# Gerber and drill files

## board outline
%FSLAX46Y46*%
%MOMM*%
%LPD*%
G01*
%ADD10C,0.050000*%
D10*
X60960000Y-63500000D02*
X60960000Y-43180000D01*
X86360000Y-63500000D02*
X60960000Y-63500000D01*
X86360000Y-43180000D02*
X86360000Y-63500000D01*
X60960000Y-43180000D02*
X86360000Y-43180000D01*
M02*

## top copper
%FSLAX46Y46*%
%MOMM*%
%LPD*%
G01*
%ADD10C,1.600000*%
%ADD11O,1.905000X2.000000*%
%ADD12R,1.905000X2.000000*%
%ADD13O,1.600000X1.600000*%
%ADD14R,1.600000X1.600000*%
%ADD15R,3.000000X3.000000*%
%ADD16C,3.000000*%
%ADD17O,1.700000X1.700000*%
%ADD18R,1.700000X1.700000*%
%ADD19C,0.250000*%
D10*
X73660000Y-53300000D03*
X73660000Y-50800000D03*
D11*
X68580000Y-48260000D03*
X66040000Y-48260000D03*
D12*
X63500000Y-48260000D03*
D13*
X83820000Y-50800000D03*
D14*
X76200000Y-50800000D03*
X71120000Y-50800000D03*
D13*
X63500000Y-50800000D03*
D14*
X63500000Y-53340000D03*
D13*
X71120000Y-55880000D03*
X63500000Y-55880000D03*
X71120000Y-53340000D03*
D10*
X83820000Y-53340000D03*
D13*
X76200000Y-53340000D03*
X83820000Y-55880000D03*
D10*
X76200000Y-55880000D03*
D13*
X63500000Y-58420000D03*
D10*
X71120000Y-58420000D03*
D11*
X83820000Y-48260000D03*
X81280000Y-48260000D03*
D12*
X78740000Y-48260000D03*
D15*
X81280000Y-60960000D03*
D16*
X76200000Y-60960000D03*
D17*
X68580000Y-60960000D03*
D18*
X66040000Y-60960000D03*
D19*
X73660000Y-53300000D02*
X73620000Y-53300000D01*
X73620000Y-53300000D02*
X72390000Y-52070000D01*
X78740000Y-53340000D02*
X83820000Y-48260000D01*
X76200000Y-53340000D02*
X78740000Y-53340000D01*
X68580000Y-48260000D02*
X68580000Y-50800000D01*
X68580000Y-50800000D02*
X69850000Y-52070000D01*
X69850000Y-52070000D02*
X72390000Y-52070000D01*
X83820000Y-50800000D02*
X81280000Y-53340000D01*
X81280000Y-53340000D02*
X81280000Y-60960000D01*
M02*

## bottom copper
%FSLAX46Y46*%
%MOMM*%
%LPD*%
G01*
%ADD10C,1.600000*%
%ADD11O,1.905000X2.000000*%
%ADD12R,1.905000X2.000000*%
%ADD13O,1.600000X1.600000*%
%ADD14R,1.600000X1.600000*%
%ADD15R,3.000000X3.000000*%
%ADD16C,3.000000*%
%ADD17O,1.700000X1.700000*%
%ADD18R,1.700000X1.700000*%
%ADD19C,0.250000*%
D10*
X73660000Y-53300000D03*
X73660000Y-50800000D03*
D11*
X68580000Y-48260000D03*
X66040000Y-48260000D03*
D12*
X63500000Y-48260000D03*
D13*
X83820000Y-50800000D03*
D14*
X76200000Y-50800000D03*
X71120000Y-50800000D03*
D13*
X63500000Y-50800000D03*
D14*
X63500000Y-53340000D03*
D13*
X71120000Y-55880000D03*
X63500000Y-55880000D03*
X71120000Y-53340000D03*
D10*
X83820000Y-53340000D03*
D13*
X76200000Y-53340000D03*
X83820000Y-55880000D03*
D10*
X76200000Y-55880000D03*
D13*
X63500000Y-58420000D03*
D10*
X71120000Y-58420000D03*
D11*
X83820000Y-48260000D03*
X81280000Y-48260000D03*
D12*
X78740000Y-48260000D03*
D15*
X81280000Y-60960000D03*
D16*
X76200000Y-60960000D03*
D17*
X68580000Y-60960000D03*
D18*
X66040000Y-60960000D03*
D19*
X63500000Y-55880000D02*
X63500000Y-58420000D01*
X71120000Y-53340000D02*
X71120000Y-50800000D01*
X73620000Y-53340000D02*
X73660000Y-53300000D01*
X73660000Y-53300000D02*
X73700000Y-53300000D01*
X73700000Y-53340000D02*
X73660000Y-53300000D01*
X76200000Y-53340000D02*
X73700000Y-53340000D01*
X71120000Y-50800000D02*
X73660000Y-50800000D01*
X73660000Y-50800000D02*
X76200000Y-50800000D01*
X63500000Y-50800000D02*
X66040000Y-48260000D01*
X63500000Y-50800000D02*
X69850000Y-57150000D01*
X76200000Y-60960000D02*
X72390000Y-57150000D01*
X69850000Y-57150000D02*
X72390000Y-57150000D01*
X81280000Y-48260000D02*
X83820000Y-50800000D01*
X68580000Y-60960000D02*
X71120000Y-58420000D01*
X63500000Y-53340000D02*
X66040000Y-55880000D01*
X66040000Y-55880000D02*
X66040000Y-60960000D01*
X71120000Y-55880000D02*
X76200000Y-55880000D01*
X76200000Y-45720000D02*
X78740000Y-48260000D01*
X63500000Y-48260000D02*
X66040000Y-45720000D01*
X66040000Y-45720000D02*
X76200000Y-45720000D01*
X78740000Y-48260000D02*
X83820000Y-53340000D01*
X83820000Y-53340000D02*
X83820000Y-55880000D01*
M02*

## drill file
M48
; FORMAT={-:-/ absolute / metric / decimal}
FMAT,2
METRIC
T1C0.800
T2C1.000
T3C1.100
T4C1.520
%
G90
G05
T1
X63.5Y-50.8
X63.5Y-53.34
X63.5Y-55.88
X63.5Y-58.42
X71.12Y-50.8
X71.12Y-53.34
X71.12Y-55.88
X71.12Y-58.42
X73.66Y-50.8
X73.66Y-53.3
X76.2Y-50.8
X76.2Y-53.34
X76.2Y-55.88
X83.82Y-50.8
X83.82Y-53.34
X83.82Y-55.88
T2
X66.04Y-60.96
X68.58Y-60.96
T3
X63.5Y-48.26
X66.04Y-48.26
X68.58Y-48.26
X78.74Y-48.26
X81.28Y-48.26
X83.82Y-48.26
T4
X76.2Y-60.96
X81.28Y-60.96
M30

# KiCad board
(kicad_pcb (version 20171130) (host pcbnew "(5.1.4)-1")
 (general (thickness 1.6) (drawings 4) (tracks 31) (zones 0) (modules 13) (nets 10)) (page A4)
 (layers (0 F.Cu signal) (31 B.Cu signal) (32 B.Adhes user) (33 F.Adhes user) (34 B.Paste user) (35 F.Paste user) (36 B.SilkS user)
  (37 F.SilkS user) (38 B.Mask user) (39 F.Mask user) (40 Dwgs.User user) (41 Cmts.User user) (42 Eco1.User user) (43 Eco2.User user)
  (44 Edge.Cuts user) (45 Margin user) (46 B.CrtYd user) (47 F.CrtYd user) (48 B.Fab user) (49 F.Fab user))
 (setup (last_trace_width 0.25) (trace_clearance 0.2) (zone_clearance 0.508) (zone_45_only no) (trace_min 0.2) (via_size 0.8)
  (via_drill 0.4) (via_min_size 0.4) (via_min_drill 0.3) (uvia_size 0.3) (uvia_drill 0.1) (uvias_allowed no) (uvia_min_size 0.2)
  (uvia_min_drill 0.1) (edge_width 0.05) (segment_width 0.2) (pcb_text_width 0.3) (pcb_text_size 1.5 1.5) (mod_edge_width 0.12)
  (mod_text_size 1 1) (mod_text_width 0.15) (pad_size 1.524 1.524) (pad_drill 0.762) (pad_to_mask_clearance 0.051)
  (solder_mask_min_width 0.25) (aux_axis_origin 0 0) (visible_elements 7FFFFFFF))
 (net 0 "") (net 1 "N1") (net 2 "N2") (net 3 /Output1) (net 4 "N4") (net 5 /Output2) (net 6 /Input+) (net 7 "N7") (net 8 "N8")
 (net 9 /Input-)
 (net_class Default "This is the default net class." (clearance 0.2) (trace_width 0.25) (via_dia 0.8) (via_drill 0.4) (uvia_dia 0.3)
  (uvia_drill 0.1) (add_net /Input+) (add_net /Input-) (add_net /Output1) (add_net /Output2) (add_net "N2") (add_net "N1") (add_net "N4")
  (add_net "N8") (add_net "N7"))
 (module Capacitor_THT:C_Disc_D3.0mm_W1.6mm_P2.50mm (layer F.Cu) (at 73.66 50.8 270)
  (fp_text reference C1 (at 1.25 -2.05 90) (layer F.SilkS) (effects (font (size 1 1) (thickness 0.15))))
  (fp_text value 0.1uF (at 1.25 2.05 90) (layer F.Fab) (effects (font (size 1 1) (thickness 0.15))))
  (pad 2 thru_hole circle (at 2.5 0 270) (size 1.6 1.6) (drill 0.8) (layers *.Cu *.Mask) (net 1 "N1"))
  (pad 1 thru_hole circle (at 0 0 270) (size 1.6 1.6) (drill 0.8) (layers *.Cu *.Mask) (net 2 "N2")))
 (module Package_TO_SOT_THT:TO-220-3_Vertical (layer F.Cu) (at 63.5 48.26)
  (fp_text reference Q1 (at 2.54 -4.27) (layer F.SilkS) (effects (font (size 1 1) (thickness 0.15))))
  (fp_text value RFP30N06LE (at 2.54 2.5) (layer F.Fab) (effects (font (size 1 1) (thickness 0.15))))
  (pad 3 thru_hole oval (at 5.08 0) (size 1.905 2) (drill 1.1) (layers *.Cu *.Mask) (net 1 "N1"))
  (pad 2 thru_hole oval (at 2.54 0) (size 1.905 2) (drill 1.1) (layers *.Cu *.Mask) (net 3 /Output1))
  (pad 1 thru_hole rect (at 0 0) (size 1.905 2) (drill 1.1) (layers *.Cu *.Mask) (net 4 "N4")))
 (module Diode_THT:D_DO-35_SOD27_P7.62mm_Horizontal (layer F.Cu) (at 76.2 50.8)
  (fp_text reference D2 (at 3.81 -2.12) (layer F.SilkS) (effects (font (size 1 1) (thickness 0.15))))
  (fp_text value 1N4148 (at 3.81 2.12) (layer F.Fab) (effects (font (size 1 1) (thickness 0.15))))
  (pad 2 thru_hole oval (at 7.62 0) (size 1.6 1.6) (drill 0.8) (layers *.Cu *.Mask) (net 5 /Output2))
  (pad 1 thru_hole rect (at 0 0) (size 1.6 1.6) (drill 0.8) (layers *.Cu *.Mask) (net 2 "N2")))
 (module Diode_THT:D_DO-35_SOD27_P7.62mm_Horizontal (layer F.Cu) (at 71.12 50.8 180)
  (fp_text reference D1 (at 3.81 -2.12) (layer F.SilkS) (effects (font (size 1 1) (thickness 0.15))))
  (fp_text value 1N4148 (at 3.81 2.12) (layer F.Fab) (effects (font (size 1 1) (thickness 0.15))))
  (pad 1 thru_hole rect (at 0 0 180) (size 1.6 1.6) (drill 0.8) (layers *.Cu *.Mask) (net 2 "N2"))
  (pad 2 thru_hole oval (at 7.62 0 180) (size 1.6 1.6) (drill 0.8) (layers *.Cu *.Mask) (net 3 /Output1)))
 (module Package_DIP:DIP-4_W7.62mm (layer F.Cu) (at 63.5 53.34)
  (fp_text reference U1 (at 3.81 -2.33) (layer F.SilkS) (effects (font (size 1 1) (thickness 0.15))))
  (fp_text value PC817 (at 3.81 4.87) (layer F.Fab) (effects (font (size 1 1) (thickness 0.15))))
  (pad 1 thru_hole rect (at 0 0) (size 1.6 1.6) (drill 0.8) (layers *.Cu *.Mask) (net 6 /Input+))
  (pad 3 thru_hole oval (at 7.62 2.54) (size 1.6 1.6) (drill 0.8) (layers *.Cu *.Mask) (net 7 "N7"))
  (pad 2 thru_hole oval (at 0 2.54) (size 1.6 1.6) (drill 0.8) (layers *.Cu *.Mask) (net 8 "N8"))
  (pad 4 thru_hole oval (at 7.62 0) (size 1.6 1.6) (drill 0.8) (layers *.Cu *.Mask) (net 2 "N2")))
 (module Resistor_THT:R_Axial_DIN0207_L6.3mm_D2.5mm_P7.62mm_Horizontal (layer F.Cu) (at 83.82 53.34 180)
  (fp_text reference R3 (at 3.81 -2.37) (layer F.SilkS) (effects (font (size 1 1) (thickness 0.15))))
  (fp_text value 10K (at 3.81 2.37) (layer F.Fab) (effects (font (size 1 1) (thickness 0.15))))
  (pad 1 thru_hole circle (at 0 0 180) (size 1.6 1.6) (drill 0.8) (layers *.Cu *.Mask) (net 4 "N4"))
  (pad 2 thru_hole oval (at 7.62 0 180) (size 1.6 1.6) (drill 0.8) (layers *.Cu *.Mask) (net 1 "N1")))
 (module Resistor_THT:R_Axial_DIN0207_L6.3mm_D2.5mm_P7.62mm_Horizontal (layer F.Cu) (at 76.2 55.88)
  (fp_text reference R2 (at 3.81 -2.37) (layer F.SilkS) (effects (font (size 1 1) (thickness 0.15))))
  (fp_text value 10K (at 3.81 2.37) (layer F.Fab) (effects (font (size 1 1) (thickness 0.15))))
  (pad 2 thru_hole oval (at 7.62 0) (size 1.6 1.6) (drill 0.8) (layers *.Cu *.Mask) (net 4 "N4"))
  (pad 1 thru_hole circle (at 0 0) (size 1.6 1.6) (drill 0.8) (layers *.Cu *.Mask) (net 7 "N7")))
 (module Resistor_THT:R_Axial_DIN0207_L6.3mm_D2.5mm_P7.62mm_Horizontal (layer F.Cu) (at 71.12 58.42 180)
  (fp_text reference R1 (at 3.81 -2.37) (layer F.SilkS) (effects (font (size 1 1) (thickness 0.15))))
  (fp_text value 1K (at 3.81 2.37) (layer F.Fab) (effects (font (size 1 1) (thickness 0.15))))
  (pad 2 thru_hole oval (at 7.62 0 180) (size 1.6 1.6) (drill 0.8) (layers *.Cu *.Mask) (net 8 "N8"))
  (pad 1 thru_hole circle (at 0 0 180) (size 1.6 1.6) (drill 0.8) (layers *.Cu *.Mask) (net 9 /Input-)))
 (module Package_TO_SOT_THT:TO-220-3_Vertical (layer F.Cu) (at 78.74 48.26)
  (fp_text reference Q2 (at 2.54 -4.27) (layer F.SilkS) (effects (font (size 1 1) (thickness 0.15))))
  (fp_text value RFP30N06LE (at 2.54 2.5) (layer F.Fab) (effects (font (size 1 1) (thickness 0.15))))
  (pad 3 thru_hole oval (at 5.08 0) (size 1.905 2) (drill 1.1) (layers *.Cu *.Mask) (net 1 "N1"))
  (pad 2 thru_hole oval (at 2.54 0) (size 1.905 2) (drill 1.1) (layers *.Cu *.Mask) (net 5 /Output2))
  (pad 1 thru_hole rect (at 0 0) (size 1.905 2) (drill 1.1) (layers *.Cu *.Mask) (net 4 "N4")))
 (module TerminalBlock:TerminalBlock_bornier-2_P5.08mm (layer F.Cu) (at 81.28 60.96 180)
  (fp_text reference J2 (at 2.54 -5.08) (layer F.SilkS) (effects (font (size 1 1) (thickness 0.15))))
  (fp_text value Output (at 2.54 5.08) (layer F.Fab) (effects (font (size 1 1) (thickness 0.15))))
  (pad 1 thru_hole rect (at 0 0 180) (size 3 3) (drill 1.52) (layers *.Cu *.Mask) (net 5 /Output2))
  (pad 2 thru_hole circle (at 5.08 0 180) (size 3 3) (drill 1.52) (layers *.Cu *.Mask) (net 3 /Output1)))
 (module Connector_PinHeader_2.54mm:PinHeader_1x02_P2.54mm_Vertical (layer F.Cu) (at 66.04 60.96 90)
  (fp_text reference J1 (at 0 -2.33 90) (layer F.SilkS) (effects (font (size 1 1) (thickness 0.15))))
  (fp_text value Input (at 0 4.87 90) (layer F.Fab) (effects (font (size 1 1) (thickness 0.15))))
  (pad 2 thru_hole oval (at 0 2.54 90) (size 1.7 1.7) (drill 1) (layers *.Cu *.Mask) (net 9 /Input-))
  (pad 1 thru_hole rect (at 0 0 90) (size 1.7 1.7) (drill 1) (layers *.Cu *.Mask) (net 6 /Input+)))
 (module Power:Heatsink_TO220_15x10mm (layer F.Cu) (at 81.28 44.45)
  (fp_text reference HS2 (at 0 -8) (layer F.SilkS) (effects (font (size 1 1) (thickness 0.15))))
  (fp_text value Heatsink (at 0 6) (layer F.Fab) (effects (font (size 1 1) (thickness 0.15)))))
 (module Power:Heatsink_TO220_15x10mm (layer F.Cu) (at 66.04 44.45)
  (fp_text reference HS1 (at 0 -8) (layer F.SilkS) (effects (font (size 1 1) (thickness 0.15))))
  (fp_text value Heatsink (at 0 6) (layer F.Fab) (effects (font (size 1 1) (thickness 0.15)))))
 (gr_line (start 60.96 63.5) (end 60.96 43.18) (layer Edge.Cuts) (width 0.05))
 (gr_line (start 86.36 63.5) (end 60.96 63.5) (layer Edge.Cuts) (width 0.05))
 (gr_line (start 86.36 43.18) (end 86.36 63.5) (layer Edge.Cuts) (width 0.05))
 (gr_line (start 60.96 43.18) (end 86.36 43.18) (layer Edge.Cuts) (width 0.05))
 (segment (start 63.5 55.88) (end 63.5 58.42) (width 0.25) (layer B.Cu) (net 8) (status 30))
 (segment (start 71.12 53.34) (end 71.12 50.8) (width 0.25) (layer B.Cu) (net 2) (status 30))
 (segment (start 73.62 53.34) (end 73.66 53.3) (width 0.25) (layer B.Cu) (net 1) (status 30))
 (segment (start 73.66 53.3) (end 73.7 53.3) (width 0.25) (layer B.Cu) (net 1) (status 30))
 (segment (start 73.7 53.34) (end 73.66 53.3) (width 0.25) (layer B.Cu) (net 1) (status 30))
 (segment (start 76.2 53.34) (end 73.7 53.34) (width 0.25) (layer B.Cu) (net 1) (status 30))
 (segment (start 73.66 53.3) (end 73.62 53.3) (width 0.25) (layer F.Cu) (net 1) (status 30))
 (segment (start 73.62 53.3) (end 72.39 52.07) (width 0.25) (layer F.Cu) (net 1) (status 10))
 (segment (start 78.74 53.34) (end 83.82 48.26) (width 0.25) (layer F.Cu) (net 1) (status 20))
 (segment (start 76.2 53.34) (end 78.74 53.34) (width 0.25) (layer F.Cu) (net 1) (status 10))
 (segment (start 68.58 48.26) (end 68.58 50.8) (width 0.25) (layer F.Cu) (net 1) (status 10))
 (segment (start 68.58 50.8) (end 69.85 52.07) (width 0.25) (layer F.Cu) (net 1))
 (segment (start 69.85 52.07) (end 72.39 52.07) (width 0.25) (layer F.Cu) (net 1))
 (segment (start 71.12 50.8) (end 73.66 50.8) (width 0.25) (layer B.Cu) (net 2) (status 30))
 (segment (start 73.66 50.8) (end 76.2 50.8) (width 0.25) (layer B.Cu) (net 2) (status 30))
 (segment (start 63.5 50.8) (end 66.04 48.26) (width 0.25) (layer B.Cu) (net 3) (status 30))
 (segment (start 63.5 50.8) (end 69.85 57.15) (width 0.25) (layer B.Cu) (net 3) (status 10))
 (segment (start 76.2 60.96) (end 72.39 57.15) (width 0.25) (layer B.Cu) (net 3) (status 10))
 (segment (start 69.85 57.15) (end 72.39 57.15) (width 0.25) (layer B.Cu) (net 3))
 (segment (start 81.28 48.26) (end 83.82 50.8) (width 0.25) (layer B.Cu) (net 5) (status 30))
 (segment (start 83.82 50.8) (end 81.28 53.34) (width 0.25) (layer F.Cu) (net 5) (status 10))
 (segment (start 81.28 53.34) (end 81.28 60.96) (width 0.25) (layer F.Cu) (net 5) (status 20))
 (segment (start 68.58 60.96) (end 71.12 58.42) (width 0.25) (layer B.Cu) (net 9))
 (segment (start 63.5 53.34) (end 66.04 55.88) (width 0.25) (layer B.Cu) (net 6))
 (segment (start 66.04 55.88) (end 66.04 60.96) (width 0.25) (layer B.Cu) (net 6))
 (segment (start 71.12 55.88) (end 76.2 55.88) (width 0.25) (layer B.Cu) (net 7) (status 30))
 (segment (start 76.2 45.72) (end 78.74 48.26) (width 0.25) (layer B.Cu) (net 4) (status 20))
 (segment (start 63.5 48.26) (end 66.04 45.72) (width 0.25) (layer B.Cu) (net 4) (status 10))
 (segment (start 66.04 45.72) (end 76.2 45.72) (width 0.25) (layer B.Cu) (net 4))
 (segment (start 78.74 48.26) (end 83.82 53.34) (width 0.25) (layer B.Cu) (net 4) (status 30))
 (segment (start 83.82 53.34) (end 83.82 55.88) (width 0.25) (layer B.Cu) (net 4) (status 30)))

